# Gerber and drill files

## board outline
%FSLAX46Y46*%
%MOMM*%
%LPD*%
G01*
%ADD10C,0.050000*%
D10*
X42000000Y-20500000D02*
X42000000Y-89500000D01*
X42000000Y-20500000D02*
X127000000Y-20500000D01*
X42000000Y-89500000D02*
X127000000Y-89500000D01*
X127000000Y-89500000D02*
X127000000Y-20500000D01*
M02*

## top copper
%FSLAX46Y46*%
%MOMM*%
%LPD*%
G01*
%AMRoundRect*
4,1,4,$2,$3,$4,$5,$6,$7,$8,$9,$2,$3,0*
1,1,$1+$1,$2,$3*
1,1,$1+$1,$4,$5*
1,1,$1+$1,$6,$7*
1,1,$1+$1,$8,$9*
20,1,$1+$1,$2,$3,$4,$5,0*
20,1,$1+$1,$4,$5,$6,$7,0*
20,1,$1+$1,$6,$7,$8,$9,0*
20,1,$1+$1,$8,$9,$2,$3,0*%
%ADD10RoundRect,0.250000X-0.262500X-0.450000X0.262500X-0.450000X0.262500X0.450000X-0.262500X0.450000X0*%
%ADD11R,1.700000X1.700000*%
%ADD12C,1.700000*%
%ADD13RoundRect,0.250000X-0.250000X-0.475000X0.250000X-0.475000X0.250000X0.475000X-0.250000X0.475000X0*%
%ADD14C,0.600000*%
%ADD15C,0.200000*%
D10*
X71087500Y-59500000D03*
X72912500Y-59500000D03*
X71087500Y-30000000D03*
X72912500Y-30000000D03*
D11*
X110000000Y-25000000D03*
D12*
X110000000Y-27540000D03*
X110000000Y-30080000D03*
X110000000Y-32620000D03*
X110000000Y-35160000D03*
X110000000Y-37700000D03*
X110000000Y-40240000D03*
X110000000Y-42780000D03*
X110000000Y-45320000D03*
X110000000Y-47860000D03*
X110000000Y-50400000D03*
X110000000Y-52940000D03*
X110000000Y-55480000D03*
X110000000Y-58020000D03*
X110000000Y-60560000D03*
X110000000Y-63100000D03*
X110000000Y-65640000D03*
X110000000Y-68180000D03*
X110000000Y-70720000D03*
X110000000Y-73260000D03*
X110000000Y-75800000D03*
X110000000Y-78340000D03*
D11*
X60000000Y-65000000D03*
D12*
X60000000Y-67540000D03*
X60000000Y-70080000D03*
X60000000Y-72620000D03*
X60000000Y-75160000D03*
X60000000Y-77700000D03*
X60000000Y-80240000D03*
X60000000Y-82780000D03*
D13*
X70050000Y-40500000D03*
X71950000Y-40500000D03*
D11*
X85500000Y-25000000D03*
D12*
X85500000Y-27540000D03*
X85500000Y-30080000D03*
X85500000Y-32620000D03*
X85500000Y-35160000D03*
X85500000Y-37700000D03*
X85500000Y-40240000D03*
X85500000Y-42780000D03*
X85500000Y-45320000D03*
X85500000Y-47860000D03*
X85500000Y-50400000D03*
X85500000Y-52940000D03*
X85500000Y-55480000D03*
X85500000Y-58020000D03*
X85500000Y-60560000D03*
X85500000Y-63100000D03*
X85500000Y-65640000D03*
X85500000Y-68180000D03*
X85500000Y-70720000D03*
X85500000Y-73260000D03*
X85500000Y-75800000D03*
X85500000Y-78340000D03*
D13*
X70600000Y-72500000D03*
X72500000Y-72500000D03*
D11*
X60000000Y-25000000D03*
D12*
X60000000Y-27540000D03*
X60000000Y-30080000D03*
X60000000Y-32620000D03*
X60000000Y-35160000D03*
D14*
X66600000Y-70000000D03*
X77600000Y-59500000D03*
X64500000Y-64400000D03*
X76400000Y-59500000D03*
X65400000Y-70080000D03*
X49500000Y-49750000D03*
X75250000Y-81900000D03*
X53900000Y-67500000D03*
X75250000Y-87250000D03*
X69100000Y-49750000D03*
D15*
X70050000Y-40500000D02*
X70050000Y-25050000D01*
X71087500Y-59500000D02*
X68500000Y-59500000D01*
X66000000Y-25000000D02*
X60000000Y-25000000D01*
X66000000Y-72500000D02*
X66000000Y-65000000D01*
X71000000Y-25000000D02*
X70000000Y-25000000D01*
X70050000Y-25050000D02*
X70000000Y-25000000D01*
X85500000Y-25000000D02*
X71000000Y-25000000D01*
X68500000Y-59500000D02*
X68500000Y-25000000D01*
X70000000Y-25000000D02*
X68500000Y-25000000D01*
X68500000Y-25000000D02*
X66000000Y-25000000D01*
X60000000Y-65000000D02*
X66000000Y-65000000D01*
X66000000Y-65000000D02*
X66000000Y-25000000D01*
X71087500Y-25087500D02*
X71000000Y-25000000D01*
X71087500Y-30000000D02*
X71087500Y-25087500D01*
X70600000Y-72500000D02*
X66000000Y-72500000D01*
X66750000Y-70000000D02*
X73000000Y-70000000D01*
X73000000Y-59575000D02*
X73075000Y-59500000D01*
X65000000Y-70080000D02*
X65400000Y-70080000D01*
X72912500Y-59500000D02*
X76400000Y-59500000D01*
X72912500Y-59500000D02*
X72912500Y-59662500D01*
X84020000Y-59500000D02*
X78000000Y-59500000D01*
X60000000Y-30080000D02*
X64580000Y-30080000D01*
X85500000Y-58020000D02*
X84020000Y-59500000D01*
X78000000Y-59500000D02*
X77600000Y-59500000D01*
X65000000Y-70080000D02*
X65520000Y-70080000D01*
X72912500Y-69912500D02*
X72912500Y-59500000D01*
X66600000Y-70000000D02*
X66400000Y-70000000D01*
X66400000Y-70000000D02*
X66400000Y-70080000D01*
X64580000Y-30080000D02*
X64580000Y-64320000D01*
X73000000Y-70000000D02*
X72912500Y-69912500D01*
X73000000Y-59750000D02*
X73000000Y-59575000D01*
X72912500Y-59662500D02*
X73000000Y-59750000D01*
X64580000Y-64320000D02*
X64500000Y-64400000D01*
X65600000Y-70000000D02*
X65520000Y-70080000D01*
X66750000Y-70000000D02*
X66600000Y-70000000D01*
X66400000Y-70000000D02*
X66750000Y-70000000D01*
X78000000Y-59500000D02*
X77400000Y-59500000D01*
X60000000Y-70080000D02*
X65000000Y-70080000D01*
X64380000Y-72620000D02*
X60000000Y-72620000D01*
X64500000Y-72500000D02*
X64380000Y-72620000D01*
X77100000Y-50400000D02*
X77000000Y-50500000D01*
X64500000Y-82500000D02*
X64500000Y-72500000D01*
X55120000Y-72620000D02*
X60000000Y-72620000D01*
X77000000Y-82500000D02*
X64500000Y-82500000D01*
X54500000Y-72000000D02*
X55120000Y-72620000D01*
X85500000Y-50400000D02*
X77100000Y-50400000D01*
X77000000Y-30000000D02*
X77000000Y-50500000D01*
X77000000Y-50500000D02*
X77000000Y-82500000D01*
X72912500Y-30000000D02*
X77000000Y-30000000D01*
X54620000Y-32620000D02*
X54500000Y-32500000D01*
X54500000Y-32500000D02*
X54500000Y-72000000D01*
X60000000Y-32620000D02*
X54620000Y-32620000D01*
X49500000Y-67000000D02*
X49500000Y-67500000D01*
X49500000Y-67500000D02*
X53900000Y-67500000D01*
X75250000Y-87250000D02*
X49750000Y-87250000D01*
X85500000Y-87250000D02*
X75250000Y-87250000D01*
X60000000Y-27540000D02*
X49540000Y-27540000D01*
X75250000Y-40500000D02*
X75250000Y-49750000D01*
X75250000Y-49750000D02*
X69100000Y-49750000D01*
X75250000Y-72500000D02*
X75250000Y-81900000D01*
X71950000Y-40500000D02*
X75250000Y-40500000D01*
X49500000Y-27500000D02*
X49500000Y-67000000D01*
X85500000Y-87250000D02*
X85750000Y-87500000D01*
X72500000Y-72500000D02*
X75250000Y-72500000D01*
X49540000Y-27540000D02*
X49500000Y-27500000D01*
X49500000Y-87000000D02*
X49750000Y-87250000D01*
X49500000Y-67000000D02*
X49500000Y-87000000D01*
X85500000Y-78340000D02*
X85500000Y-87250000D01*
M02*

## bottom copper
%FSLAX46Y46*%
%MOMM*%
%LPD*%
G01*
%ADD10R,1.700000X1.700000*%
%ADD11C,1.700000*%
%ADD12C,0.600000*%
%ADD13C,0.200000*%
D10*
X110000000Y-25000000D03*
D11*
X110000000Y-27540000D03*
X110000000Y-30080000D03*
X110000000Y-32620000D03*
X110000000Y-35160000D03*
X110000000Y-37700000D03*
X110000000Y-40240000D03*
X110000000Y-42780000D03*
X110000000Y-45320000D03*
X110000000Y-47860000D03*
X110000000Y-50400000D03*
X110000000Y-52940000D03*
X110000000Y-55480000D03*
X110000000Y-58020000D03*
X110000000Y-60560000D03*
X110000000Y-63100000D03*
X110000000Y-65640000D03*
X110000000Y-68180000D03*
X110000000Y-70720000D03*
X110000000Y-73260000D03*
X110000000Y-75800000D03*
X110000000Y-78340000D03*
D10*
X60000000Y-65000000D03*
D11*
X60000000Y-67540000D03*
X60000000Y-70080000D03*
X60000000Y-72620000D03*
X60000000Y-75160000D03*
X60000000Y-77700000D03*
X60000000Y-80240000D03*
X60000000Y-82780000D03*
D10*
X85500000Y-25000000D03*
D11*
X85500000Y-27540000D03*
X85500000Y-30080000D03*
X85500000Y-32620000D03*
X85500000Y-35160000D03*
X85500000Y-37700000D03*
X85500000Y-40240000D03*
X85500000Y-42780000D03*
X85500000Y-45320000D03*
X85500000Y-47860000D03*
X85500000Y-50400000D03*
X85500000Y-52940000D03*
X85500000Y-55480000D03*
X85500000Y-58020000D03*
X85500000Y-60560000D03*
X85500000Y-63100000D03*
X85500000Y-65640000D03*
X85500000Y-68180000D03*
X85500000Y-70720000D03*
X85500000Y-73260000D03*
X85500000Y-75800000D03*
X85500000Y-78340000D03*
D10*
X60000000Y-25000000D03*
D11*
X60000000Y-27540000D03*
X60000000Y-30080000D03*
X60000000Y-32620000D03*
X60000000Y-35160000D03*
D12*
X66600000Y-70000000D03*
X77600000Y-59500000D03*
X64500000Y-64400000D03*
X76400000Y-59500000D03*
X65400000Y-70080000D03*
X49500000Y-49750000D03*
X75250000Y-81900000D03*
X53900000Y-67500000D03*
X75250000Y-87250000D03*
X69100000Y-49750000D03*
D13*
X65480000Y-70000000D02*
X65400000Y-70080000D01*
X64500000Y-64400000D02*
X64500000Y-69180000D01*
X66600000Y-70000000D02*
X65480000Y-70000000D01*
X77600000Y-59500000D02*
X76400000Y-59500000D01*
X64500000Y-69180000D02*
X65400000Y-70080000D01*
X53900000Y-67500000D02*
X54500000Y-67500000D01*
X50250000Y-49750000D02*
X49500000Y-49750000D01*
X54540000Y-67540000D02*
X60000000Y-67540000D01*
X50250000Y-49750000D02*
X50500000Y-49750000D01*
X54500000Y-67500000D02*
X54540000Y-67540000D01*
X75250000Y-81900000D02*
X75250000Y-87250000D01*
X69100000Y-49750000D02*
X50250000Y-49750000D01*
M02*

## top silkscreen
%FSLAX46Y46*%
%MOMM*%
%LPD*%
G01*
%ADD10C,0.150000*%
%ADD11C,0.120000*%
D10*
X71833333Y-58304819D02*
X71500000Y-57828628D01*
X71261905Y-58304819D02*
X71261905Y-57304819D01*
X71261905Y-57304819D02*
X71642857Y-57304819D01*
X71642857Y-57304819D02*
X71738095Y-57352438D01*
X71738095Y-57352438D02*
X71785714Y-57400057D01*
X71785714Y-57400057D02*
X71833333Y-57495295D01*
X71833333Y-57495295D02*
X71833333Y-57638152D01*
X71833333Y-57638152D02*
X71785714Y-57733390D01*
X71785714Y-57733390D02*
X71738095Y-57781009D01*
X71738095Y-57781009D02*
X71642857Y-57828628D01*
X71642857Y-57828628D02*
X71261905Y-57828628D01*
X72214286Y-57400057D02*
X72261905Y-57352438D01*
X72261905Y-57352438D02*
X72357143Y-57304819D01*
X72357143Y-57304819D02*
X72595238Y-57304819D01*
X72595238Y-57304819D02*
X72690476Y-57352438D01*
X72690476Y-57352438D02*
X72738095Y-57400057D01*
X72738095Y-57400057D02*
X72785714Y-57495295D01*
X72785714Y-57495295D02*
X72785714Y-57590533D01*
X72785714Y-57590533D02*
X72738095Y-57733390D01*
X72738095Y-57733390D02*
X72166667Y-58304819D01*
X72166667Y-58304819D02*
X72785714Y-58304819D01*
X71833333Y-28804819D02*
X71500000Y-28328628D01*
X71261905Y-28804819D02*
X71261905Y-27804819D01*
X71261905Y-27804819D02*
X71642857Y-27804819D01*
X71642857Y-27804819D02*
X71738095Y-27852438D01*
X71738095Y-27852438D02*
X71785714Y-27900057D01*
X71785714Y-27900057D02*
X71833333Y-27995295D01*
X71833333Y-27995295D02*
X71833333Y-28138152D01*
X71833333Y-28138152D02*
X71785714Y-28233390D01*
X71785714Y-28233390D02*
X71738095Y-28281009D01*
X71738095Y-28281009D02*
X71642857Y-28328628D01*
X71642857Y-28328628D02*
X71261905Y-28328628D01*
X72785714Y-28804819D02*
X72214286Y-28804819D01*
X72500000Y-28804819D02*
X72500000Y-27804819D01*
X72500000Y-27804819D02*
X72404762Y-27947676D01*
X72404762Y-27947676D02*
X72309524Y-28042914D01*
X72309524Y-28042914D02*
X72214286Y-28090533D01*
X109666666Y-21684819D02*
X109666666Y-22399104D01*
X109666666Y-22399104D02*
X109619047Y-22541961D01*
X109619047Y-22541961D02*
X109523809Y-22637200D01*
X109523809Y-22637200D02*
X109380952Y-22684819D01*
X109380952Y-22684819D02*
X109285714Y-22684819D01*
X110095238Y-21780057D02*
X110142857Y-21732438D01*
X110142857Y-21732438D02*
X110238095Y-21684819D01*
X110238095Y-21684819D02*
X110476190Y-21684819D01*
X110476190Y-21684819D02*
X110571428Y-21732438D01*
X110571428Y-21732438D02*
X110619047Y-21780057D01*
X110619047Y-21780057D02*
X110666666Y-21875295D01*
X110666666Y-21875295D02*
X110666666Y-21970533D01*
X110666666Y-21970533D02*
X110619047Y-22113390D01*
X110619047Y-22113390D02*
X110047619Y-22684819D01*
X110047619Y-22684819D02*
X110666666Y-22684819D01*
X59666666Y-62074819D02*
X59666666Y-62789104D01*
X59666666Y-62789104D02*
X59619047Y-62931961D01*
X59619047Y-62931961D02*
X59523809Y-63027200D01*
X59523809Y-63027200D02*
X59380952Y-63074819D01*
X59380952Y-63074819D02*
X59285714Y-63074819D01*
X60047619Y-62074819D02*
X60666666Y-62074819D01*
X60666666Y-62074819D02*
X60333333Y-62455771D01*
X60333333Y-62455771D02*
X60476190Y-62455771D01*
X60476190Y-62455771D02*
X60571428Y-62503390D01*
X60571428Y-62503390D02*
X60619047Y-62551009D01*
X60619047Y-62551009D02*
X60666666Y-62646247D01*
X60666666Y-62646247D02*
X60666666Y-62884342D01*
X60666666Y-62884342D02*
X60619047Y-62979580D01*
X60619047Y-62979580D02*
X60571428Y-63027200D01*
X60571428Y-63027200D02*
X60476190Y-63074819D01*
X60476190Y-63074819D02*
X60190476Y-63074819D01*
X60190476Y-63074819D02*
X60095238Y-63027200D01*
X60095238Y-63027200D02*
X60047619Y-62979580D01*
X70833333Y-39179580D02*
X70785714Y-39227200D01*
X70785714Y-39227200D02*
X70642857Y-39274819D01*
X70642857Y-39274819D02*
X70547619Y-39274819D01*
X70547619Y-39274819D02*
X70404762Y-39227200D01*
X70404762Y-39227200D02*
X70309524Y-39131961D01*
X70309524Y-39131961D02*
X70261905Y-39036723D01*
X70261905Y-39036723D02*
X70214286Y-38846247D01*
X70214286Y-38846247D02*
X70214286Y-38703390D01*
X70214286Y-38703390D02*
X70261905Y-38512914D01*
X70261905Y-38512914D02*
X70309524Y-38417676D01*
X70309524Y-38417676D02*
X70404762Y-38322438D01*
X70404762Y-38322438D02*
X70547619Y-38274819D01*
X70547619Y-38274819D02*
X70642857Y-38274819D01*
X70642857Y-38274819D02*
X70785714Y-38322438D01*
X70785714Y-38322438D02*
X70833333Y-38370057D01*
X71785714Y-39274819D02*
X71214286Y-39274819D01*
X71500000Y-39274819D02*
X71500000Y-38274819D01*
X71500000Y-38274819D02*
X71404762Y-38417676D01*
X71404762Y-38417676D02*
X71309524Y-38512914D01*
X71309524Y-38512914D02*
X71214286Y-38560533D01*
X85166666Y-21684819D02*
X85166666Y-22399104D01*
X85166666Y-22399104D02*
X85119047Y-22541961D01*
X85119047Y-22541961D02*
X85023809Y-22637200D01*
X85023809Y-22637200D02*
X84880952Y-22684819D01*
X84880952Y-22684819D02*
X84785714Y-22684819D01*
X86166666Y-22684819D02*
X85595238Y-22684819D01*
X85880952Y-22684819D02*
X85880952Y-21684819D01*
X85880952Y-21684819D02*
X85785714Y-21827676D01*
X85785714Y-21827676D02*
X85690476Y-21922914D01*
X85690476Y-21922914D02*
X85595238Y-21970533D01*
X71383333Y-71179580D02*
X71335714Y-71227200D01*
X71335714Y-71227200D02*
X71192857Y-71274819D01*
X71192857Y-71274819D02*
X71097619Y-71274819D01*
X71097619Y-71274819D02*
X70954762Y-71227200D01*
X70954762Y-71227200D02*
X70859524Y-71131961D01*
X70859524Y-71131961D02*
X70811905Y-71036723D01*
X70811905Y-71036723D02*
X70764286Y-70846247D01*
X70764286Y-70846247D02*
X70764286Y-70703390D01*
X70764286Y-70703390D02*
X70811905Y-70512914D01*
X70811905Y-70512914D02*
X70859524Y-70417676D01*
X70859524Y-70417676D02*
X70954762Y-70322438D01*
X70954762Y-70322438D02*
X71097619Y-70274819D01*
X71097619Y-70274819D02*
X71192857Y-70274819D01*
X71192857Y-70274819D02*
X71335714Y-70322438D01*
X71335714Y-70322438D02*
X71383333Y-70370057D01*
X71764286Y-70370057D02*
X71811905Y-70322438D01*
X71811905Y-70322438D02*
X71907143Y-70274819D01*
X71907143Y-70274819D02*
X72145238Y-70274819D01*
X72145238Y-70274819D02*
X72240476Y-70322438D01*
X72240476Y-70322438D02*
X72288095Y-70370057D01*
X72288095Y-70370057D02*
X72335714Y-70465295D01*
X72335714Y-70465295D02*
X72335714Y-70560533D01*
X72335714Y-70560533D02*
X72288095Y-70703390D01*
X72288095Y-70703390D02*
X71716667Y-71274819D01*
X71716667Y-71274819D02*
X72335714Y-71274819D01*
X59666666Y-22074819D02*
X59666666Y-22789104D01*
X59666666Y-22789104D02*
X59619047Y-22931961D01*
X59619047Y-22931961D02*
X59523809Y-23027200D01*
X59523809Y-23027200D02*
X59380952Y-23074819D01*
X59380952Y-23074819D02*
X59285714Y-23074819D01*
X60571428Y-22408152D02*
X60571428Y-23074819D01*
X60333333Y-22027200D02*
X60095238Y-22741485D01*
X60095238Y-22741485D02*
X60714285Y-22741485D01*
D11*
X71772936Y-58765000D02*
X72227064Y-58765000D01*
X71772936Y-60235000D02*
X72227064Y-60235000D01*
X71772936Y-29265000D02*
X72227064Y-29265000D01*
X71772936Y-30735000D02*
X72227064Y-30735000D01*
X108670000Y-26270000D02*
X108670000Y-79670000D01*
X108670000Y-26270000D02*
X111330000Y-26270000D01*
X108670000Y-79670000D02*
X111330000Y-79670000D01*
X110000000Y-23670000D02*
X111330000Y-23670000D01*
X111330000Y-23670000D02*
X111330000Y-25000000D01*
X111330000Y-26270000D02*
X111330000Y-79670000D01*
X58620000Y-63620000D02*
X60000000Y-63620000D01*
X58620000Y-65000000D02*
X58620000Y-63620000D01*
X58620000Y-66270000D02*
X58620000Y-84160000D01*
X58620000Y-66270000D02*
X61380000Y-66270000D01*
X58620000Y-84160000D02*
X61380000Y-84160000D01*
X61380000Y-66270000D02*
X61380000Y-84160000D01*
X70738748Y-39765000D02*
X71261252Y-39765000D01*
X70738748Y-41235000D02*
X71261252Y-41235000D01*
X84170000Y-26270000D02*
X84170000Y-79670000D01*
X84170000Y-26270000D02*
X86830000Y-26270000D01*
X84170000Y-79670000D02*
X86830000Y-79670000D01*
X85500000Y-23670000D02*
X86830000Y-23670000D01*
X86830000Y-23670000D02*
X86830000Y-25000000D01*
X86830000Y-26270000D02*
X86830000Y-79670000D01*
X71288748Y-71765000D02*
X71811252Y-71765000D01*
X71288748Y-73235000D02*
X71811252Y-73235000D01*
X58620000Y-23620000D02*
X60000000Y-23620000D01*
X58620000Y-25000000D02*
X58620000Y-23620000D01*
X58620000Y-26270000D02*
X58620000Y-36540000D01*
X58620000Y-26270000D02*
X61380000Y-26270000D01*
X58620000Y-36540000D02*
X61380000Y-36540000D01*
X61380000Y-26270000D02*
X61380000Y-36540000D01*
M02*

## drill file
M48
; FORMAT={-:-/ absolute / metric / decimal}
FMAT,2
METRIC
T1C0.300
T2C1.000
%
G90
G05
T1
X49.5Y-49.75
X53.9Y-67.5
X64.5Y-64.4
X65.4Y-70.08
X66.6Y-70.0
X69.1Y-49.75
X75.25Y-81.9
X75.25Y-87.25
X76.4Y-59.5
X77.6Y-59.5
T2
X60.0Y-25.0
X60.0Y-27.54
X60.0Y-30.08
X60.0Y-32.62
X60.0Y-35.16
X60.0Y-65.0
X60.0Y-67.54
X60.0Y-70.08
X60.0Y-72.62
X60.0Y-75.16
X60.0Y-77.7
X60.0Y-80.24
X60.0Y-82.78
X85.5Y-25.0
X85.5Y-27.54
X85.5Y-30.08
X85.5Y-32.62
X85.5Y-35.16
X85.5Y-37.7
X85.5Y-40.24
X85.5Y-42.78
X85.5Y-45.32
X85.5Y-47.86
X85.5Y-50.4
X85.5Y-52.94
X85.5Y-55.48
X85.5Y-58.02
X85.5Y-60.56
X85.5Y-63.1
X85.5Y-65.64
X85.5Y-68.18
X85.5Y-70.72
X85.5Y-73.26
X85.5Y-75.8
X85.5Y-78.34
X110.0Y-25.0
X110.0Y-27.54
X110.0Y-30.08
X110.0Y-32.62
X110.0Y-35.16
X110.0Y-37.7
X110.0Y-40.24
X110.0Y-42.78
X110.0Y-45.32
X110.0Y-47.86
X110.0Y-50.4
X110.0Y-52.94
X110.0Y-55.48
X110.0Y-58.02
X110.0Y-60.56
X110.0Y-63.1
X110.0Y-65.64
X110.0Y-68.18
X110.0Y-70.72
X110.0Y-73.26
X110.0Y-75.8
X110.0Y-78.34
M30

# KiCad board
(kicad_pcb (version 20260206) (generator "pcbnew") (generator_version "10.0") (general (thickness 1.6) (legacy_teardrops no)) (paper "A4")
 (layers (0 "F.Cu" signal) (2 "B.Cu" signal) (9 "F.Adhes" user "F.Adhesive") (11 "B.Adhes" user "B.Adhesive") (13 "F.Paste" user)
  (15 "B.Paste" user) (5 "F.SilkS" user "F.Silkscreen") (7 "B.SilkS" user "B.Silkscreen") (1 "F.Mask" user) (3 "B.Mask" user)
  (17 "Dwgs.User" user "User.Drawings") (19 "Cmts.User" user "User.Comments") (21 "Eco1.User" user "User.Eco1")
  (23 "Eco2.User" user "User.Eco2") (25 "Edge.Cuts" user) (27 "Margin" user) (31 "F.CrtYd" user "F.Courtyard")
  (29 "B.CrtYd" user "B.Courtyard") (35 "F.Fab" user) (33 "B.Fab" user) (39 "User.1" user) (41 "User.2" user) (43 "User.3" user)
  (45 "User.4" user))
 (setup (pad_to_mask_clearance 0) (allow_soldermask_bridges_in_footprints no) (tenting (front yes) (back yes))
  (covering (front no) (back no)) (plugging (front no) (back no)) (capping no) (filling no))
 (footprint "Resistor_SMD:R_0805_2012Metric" (layer "F.Cu") (at 72 59.5)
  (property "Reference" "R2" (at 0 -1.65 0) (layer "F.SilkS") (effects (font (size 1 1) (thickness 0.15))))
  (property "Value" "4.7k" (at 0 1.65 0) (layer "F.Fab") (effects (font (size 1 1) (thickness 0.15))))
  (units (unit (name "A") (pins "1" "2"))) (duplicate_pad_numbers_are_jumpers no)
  (fp_line (start -0.227064 -0.735) (end 0.227064 -0.735) (stroke (width 0.12) (type solid)) (layer "F.SilkS"))
  (fp_line (start -0.227064 0.735) (end 0.227064 0.735) (stroke (width 0.12) (type solid)) (layer "F.SilkS"))
  (pad "1" smd roundrect (at -0.9125 0) (size 1.025 1.4) (layers "F.Cu" "F.Mask" "F.Paste") (roundrect_rratio 0.243902) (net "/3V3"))
  (pad "2" smd roundrect (at 0.9125 0) (size 1.025 1.4) (layers "F.Cu" "F.Mask" "F.Paste") (roundrect_rratio 0.243902) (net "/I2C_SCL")))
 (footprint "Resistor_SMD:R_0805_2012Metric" (layer "F.Cu") (at 72 30)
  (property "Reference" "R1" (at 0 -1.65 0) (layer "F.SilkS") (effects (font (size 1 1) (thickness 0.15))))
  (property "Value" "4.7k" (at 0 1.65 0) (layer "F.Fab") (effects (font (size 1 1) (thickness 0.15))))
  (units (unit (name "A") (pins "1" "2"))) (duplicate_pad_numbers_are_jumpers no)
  (fp_line (start -0.227064 -0.735) (end 0.227064 -0.735) (stroke (width 0.12) (type solid)) (layer "F.SilkS"))
  (fp_line (start -0.227064 0.735) (end 0.227064 0.735) (stroke (width 0.12) (type solid)) (layer "F.SilkS"))
  (pad "1" smd roundrect (at -0.9125 0) (size 1.025 1.4) (layers "F.Cu" "F.Mask" "F.Paste") (roundrect_rratio 0.243902) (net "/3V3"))
  (pad "2" smd roundrect (at 0.9125 0) (size 1.025 1.4) (layers "F.Cu" "F.Mask" "F.Paste") (roundrect_rratio 0.243902) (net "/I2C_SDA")))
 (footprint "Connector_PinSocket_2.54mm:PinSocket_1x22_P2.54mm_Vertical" (layer "F.Cu") (at 110 25)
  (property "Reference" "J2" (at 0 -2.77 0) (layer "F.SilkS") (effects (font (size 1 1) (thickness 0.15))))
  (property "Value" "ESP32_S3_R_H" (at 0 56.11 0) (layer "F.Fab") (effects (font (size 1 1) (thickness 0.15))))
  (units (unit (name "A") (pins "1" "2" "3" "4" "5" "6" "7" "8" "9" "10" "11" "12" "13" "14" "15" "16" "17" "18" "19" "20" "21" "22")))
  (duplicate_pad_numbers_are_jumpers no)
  (fp_line (start -1.33 1.27) (end -1.33 54.67) (stroke (width 0.12) (type solid)) (layer "F.SilkS"))
  (fp_line (start -1.33 1.27) (end 1.33 1.27) (stroke (width 0.12) (type solid)) (layer "F.SilkS"))
  (fp_line (start -1.33 54.67) (end 1.33 54.67) (stroke (width 0.12) (type solid)) (layer "F.SilkS"))
  (fp_line (start 0 -1.33) (end 1.33 -1.33) (stroke (width 0.12) (type solid)) (layer "F.SilkS"))
  (fp_line (start 1.33 -1.33) (end 1.33 0) (stroke (width 0.12) (type solid)) (layer "F.SilkS"))
  (fp_line (start 1.33 1.27) (end 1.33 54.67) (stroke (width 0.12) (type solid)) (layer "F.SilkS"))
  (pad "1" thru_hole rect (at 0 0) (size 1.7 1.7) (drill 1) (layers "*.Cu" "*.Mask") (remove_unused_layers no) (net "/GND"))
  (pad "2" thru_hole circle (at 0 2.54) (size 1.7 1.7) (drill 1) (layers "*.Cu" "*.Mask") (remove_unused_layers no)
   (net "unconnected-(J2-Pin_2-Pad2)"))
  (pad "3" thru_hole circle (at 0 5.08) (size 1.7 1.7) (drill 1) (layers "*.Cu" "*.Mask") (remove_unused_layers no)
   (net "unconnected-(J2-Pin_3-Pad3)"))
  (pad "4" thru_hole circle (at 0 7.62) (size 1.7 1.7) (drill 1) (layers "*.Cu" "*.Mask") (remove_unused_layers no)
   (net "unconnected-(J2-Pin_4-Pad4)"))
  (pad "5" thru_hole circle (at 0 10.16) (size 1.7 1.7) (drill 1) (layers "*.Cu" "*.Mask") (remove_unused_layers no)
   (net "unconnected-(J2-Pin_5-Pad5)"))
  (pad "6" thru_hole circle (at 0 12.7) (size 1.7 1.7) (drill 1) (layers "*.Cu" "*.Mask") (remove_unused_layers no)
   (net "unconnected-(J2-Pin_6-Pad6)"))
  (pad "7" thru_hole circle (at 0 15.24) (size 1.7 1.7) (drill 1) (layers "*.Cu" "*.Mask") (remove_unused_layers no)
   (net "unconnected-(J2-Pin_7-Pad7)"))
  (pad "8" thru_hole circle (at 0 17.78) (size 1.7 1.7) (drill 1) (layers "*.Cu" "*.Mask") (remove_unused_layers no)
   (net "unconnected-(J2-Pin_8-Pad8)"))
  (pad "9" thru_hole circle (at 0 20.32) (size 1.7 1.7) (drill 1) (layers "*.Cu" "*.Mask") (remove_unused_layers no)
   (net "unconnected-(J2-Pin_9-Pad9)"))
  (pad "10" thru_hole circle (at 0 22.86) (size 1.7 1.7) (drill 1) (layers "*.Cu" "*.Mask") (remove_unused_layers no)
   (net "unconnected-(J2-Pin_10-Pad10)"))
  (pad "11" thru_hole circle (at 0 25.4) (size 1.7 1.7) (drill 1) (layers "*.Cu" "*.Mask") (remove_unused_layers no)
   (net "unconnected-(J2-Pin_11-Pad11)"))
  (pad "12" thru_hole circle (at 0 27.94) (size 1.7 1.7) (drill 1) (layers "*.Cu" "*.Mask") (remove_unused_layers no)
   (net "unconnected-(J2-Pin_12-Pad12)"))
  (pad "13" thru_hole circle (at 0 30.48) (size 1.7 1.7) (drill 1) (layers "*.Cu" "*.Mask") (remove_unused_layers no)
   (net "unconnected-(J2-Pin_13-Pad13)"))
  (pad "14" thru_hole circle (at 0 33.02) (size 1.7 1.7) (drill 1) (layers "*.Cu" "*.Mask") (remove_unused_layers no)
   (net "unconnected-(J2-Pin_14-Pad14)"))
  (pad "15" thru_hole circle (at 0 35.56) (size 1.7 1.7) (drill 1) (layers "*.Cu" "*.Mask") (remove_unused_layers no)
   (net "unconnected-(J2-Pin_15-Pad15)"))
  (pad "16" thru_hole circle (at 0 38.1) (size 1.7 1.7) (drill 1) (layers "*.Cu" "*.Mask") (remove_unused_layers no)
   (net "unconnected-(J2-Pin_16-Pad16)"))
  (pad "17" thru_hole circle (at 0 40.64) (size 1.7 1.7) (drill 1) (layers "*.Cu" "*.Mask") (remove_unused_layers no)
   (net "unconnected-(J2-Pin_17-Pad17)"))
  (pad "18" thru_hole circle (at 0 43.18) (size 1.7 1.7) (drill 1) (layers "*.Cu" "*.Mask") (remove_unused_layers no)
   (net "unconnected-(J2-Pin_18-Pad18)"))
  (pad "19" thru_hole circle (at 0 45.72) (size 1.7 1.7) (drill 1) (layers "*.Cu" "*.Mask") (remove_unused_layers no)
   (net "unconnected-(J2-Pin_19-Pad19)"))
  (pad "20" thru_hole circle (at 0 48.26) (size 1.7 1.7) (drill 1) (layers "*.Cu" "*.Mask") (remove_unused_layers no)
   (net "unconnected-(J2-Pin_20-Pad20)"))
  (pad "21" thru_hole circle (at 0 50.8) (size 1.7 1.7) (drill 1) (layers "*.Cu" "*.Mask") (remove_unused_layers no) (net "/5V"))
  (pad "22" thru_hole circle (at 0 53.34) (size 1.7 1.7) (drill 1) (layers "*.Cu" "*.Mask") (remove_unused_layers no) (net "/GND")))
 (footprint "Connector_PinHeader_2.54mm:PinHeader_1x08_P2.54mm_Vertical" (layer "F.Cu") (at 60 65)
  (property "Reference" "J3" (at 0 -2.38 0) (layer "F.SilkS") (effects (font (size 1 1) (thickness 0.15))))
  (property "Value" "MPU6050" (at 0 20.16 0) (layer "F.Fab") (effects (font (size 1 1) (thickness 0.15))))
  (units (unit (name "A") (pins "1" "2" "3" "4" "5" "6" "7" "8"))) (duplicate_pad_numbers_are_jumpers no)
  (fp_line (start -1.38 -1.38) (end 0 -1.38) (stroke (width 0.12) (type solid)) (layer "F.SilkS"))
  (fp_line (start -1.38 0) (end -1.38 -1.38) (stroke (width 0.12) (type solid)) (layer "F.SilkS"))
  (fp_line (start -1.38 1.27) (end -1.38 19.16) (stroke (width 0.12) (type solid)) (layer "F.SilkS"))
  (fp_line (start -1.38 1.27) (end 1.38 1.27) (stroke (width 0.12) (type solid)) (layer "F.SilkS"))
  (fp_line (start -1.38 19.16) (end 1.38 19.16) (stroke (width 0.12) (type solid)) (layer "F.SilkS"))
  (fp_line (start 1.38 1.27) (end 1.38 19.16) (stroke (width 0.12) (type solid)) (layer "F.SilkS"))
  (pad "1" thru_hole rect (at 0 0) (size 1.7 1.7) (drill 1) (layers "*.Cu" "*.Mask") (remove_unused_layers no) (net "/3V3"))
  (pad "2" thru_hole circle (at 0 2.54) (size 1.7 1.7) (drill 1) (layers "*.Cu" "*.Mask") (remove_unused_layers no) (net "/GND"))
  (pad "3" thru_hole circle (at 0 5.08) (size 1.7 1.7) (drill 1) (layers "*.Cu" "*.Mask") (remove_unused_layers no) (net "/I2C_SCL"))
  (pad "4" thru_hole circle (at 0 7.62) (size 1.7 1.7) (drill 1) (layers "*.Cu" "*.Mask") (remove_unused_layers no) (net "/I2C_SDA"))
  (pad "5" thru_hole circle (at 0 10.16) (size 1.7 1.7) (drill 1) (layers "*.Cu" "*.Mask") (remove_unused_layers no)
   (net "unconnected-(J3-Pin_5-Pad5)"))
  (pad "6" thru_hole circle (at 0 12.7) (size 1.7 1.7) (drill 1) (layers "*.Cu" "*.Mask") (remove_unused_layers no)
   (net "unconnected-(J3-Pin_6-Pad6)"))
  (pad "7" thru_hole circle (at 0 15.24) (size 1.7 1.7) (drill 1) (layers "*.Cu" "*.Mask") (remove_unused_layers no) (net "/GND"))
  (pad "8" thru_hole circle (at 0 17.78) (size 1.7 1.7) (drill 1) (layers "*.Cu" "*.Mask") (remove_unused_layers no) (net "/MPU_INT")))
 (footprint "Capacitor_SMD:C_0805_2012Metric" (layer "F.Cu") (at 71 40.5)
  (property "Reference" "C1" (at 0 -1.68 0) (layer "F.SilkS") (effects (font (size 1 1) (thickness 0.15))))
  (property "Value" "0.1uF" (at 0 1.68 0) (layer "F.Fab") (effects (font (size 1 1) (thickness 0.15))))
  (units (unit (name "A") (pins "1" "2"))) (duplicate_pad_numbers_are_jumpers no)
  (fp_line (start -0.261252 -0.735) (end 0.261252 -0.735) (stroke (width 0.12) (type solid)) (layer "F.SilkS"))
  (fp_line (start -0.261252 0.735) (end 0.261252 0.735) (stroke (width 0.12) (type solid)) (layer "F.SilkS"))
  (pad "1" smd roundrect (at -0.95 0) (size 1 1.45) (layers "F.Cu" "F.Mask" "F.Paste") (roundrect_rratio 0.25) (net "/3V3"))
  (pad "2" smd roundrect (at 0.95 0) (size 1 1.45) (layers "F.Cu" "F.Mask" "F.Paste") (roundrect_rratio 0.25) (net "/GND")))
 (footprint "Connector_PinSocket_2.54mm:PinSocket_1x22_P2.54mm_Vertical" (layer "F.Cu") (at 85.5 25)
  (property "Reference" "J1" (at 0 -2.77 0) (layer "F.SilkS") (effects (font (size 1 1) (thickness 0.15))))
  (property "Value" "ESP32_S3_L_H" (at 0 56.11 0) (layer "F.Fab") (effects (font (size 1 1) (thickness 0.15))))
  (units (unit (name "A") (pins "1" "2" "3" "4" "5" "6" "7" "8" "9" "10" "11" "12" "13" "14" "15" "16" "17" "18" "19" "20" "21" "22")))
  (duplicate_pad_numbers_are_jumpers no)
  (fp_line (start -1.33 1.27) (end -1.33 54.67) (stroke (width 0.12) (type solid)) (layer "F.SilkS"))
  (fp_line (start -1.33 1.27) (end 1.33 1.27) (stroke (width 0.12) (type solid)) (layer "F.SilkS"))
  (fp_line (start -1.33 54.67) (end 1.33 54.67) (stroke (width 0.12) (type solid)) (layer "F.SilkS"))
  (fp_line (start 0 -1.33) (end 1.33 -1.33) (stroke (width 0.12) (type solid)) (layer "F.SilkS"))
  (fp_line (start 1.33 -1.33) (end 1.33 0) (stroke (width 0.12) (type solid)) (layer "F.SilkS"))
  (fp_line (start 1.33 1.27) (end 1.33 54.67) (stroke (width 0.12) (type solid)) (layer "F.SilkS"))
  (pad "1" thru_hole rect (at 0 0) (size 1.7 1.7) (drill 1) (layers "*.Cu" "*.Mask") (remove_unused_layers no) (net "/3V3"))
  (pad "2" thru_hole circle (at 0 2.54) (size 1.7 1.7) (drill 1) (layers "*.Cu" "*.Mask") (remove_unused_layers no)
   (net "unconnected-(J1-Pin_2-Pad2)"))
  (pad "3" thru_hole circle (at 0 5.08) (size 1.7 1.7) (drill 1) (layers "*.Cu" "*.Mask") (remove_unused_layers no)
   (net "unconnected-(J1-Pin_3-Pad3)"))
  (pad "4" thru_hole circle (at 0 7.62) (size 1.7 1.7) (drill 1) (layers "*.Cu" "*.Mask") (remove_unused_layers no)
   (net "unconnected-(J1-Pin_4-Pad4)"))
  (pad "5" thru_hole circle (at 0 10.16) (size 1.7 1.7) (drill 1) (layers "*.Cu" "*.Mask") (remove_unused_layers no)
   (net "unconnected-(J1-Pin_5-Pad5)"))
  (pad "6" thru_hole circle (at 0 12.7) (size 1.7 1.7) (drill 1) (layers "*.Cu" "*.Mask") (remove_unused_layers no)
   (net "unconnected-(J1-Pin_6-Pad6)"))
  (pad "7" thru_hole circle (at 0 15.24) (size 1.7 1.7) (drill 1) (layers "*.Cu" "*.Mask") (remove_unused_layers no)
   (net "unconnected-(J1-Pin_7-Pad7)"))
  (pad "8" thru_hole circle (at 0 17.78) (size 1.7 1.7) (drill 1) (layers "*.Cu" "*.Mask") (remove_unused_layers no)
   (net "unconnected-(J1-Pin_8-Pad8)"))
  (pad "9" thru_hole circle (at 0 20.32) (size 1.7 1.7) (drill 1) (layers "*.Cu" "*.Mask") (remove_unused_layers no)
   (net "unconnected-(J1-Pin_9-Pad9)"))
  (pad "10" thru_hole circle (at 0 22.86) (size 1.7 1.7) (drill 1) (layers "*.Cu" "*.Mask") (remove_unused_layers no)
   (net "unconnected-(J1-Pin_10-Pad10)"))
  (pad "11" thru_hole circle (at 0 25.4) (size 1.7 1.7) (drill 1) (layers "*.Cu" "*.Mask") (remove_unused_layers no) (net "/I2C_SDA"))
  (pad "12" thru_hole circle (at 0 27.94) (size 1.7 1.7) (drill 1) (layers "*.Cu" "*.Mask") (remove_unused_layers no)
   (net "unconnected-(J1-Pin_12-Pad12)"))
  (pad "13" thru_hole circle (at 0 30.48) (size 1.7 1.7) (drill 1) (layers "*.Cu" "*.Mask") (remove_unused_layers no)
   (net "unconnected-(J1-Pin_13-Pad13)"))
  (pad "14" thru_hole circle (at 0 33.02) (size 1.7 1.7) (drill 1) (layers "*.Cu" "*.Mask") (remove_unused_layers no) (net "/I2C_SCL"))
  (pad "15" thru_hole circle (at 0 35.56) (size 1.7 1.7) (drill 1) (layers "*.Cu" "*.Mask") (remove_unused_layers no) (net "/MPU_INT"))
  (pad "16" thru_hole circle (at 0 38.1) (size 1.7 1.7) (drill 1) (layers "*.Cu" "*.Mask") (remove_unused_layers no) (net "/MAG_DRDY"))
  (pad "17" thru_hole circle (at 0 40.64) (size 1.7 1.7) (drill 1) (layers "*.Cu" "*.Mask") (remove_unused_layers no)
   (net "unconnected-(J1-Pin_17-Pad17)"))
  (pad "18" thru_hole circle (at 0 43.18) (size 1.7 1.7) (drill 1) (layers "*.Cu" "*.Mask") (remove_unused_layers no)
   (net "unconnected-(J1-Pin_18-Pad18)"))
  (pad "19" thru_hole circle (at 0 45.72) (size 1.7 1.7) (drill 1) (layers "*.Cu" "*.Mask") (remove_unused_layers no)
   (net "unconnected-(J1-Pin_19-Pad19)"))
  (pad "20" thru_hole circle (at 0 48.26) (size 1.7 1.7) (drill 1) (layers "*.Cu" "*.Mask") (remove_unused_layers no)
   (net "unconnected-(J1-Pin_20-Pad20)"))
  (pad "21" thru_hole circle (at 0 50.8) (size 1.7 1.7) (drill 1) (layers "*.Cu" "*.Mask") (remove_unused_layers no) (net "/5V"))
  (pad "22" thru_hole circle (at 0 53.34) (size 1.7 1.7) (drill 1) (layers "*.Cu" "*.Mask") (remove_unused_layers no) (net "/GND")))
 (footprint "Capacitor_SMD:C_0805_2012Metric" (layer "F.Cu") (at 71.55 72.5)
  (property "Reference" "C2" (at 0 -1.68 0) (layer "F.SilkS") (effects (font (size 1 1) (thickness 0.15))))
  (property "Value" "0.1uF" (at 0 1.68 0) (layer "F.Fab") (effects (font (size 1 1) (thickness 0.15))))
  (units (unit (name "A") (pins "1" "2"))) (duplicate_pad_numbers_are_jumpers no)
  (fp_line (start -0.261252 -0.735) (end 0.261252 -0.735) (stroke (width 0.12) (type solid)) (layer "F.SilkS"))
  (fp_line (start -0.261252 0.735) (end 0.261252 0.735) (stroke (width 0.12) (type solid)) (layer "F.SilkS"))
  (pad "1" smd roundrect (at -0.95 0) (size 1 1.45) (layers "F.Cu" "F.Mask" "F.Paste") (roundrect_rratio 0.25) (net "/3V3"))
  (pad "2" smd roundrect (at 0.95 0) (size 1 1.45) (layers "F.Cu" "F.Mask" "F.Paste") (roundrect_rratio 0.25) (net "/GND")))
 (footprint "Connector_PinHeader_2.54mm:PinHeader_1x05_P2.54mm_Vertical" (layer "F.Cu") (at 60 25)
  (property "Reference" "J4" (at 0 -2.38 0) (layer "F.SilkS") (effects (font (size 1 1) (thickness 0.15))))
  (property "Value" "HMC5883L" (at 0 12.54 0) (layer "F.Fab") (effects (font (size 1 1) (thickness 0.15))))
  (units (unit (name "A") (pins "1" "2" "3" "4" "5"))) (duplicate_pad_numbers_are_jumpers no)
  (fp_line (start -1.38 -1.38) (end 0 -1.38) (stroke (width 0.12) (type solid)) (layer "F.SilkS"))
  (fp_line (start -1.38 0) (end -1.38 -1.38) (stroke (width 0.12) (type solid)) (layer "F.SilkS"))
  (fp_line (start -1.38 1.27) (end -1.38 11.54) (stroke (width 0.12) (type solid)) (layer "F.SilkS"))
  (fp_line (start -1.38 1.27) (end 1.38 1.27) (stroke (width 0.12) (type solid)) (layer "F.SilkS"))
  (fp_line (start -1.38 11.54) (end 1.38 11.54) (stroke (width 0.12) (type solid)) (layer "F.SilkS"))
  (fp_line (start 1.38 1.27) (end 1.38 11.54) (stroke (width 0.12) (type solid)) (layer "F.SilkS"))
  (pad "1" thru_hole rect (at 0 0) (size 1.7 1.7) (drill 1) (layers "*.Cu" "*.Mask") (remove_unused_layers no) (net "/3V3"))
  (pad "2" thru_hole circle (at 0 2.54) (size 1.7 1.7) (drill 1) (layers "*.Cu" "*.Mask") (remove_unused_layers no) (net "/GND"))
  (pad "3" thru_hole circle (at 0 5.08) (size 1.7 1.7) (drill 1) (layers "*.Cu" "*.Mask") (remove_unused_layers no) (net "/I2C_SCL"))
  (pad "4" thru_hole circle (at 0 7.62) (size 1.7 1.7) (drill 1) (layers "*.Cu" "*.Mask") (remove_unused_layers no) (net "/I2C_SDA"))
  (pad "5" thru_hole circle (at 0 10.16) (size 1.7 1.7) (drill 1) (layers "*.Cu" "*.Mask") (remove_unused_layers no) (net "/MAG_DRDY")))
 (gr_line (start 42 20.5) (end 42 89.5) (stroke (width 0.05) (type default)) (layer "Edge.Cuts"))
 (gr_line (start 42 20.5) (end 127 20.5) (stroke (width 0.05) (type default)) (layer "Edge.Cuts"))
 (gr_line (start 42 89.5) (end 127 89.5) (stroke (width 0.05) (type default)) (layer "Edge.Cuts"))
 (gr_line (start 127 89.5) (end 127 20.5) (stroke (width 0.05) (type default)) (layer "Edge.Cuts"))
 (segment (start 70.05 40.5) (end 70.05 25.05) (width 0.2) (layer "F.Cu") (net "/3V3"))
 (segment (start 71.0875 59.5) (end 68.5 59.5) (width 0.2) (layer "F.Cu") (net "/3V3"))
 (segment (start 66 25) (end 60 25) (width 0.2) (layer "F.Cu") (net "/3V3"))
 (segment (start 66 72.5) (end 66 65) (width 0.2) (layer "F.Cu") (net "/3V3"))
 (segment (start 71 25) (end 70 25) (width 0.2) (layer "F.Cu") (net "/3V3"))
 (segment (start 70.05 25.05) (end 70 25) (width 0.2) (layer "F.Cu") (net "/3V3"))
 (segment (start 85.5 25) (end 71 25) (width 0.2) (layer "F.Cu") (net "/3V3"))
 (segment (start 68.5 59.5) (end 68.5 25) (width 0.2) (layer "F.Cu") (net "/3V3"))
 (segment (start 70 25) (end 68.5 25) (width 0.2) (layer "F.Cu") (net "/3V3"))
 (segment (start 68.5 25) (end 66 25) (width 0.2) (layer "F.Cu") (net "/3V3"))
 (segment (start 60 65) (end 66 65) (width 0.2) (layer "F.Cu") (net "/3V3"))
 (segment (start 66 65) (end 66 25) (width 0.2) (layer "F.Cu") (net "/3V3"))
 (segment (start 71.0875 25.0875) (end 71 25) (width 0.2) (layer "F.Cu") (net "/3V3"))
 (segment (start 71.0875 30) (end 71.0875 25.0875) (width 0.2) (layer "F.Cu") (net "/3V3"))
 (segment (start 70.6 72.5) (end 66 72.5) (width 0.2) (layer "F.Cu") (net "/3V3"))
 (segment (start 66.75 70) (end 73 70) (width 0.2) (layer "F.Cu") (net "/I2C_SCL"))
 (segment (start 73 59.575) (end 73.075 59.5) (width 0.2) (layer "F.Cu") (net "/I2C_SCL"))
 (segment (start 65 70.08) (end 65.4 70.08) (width 0.2) (layer "F.Cu") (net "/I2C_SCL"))
 (segment (start 72.9125 59.5) (end 76.4 59.5) (width 0.2) (layer "F.Cu") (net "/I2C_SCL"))
 (segment (start 72.9125 59.5) (end 72.9125 59.6625) (width 0.2) (layer "F.Cu") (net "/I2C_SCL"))
 (segment (start 84.02 59.5) (end 78 59.5) (width 0.2) (layer "F.Cu") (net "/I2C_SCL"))
 (segment (start 60 30.08) (end 64.58 30.08) (width 0.2) (layer "F.Cu") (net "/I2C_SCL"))
 (segment (start 85.5 58.02) (end 84.02 59.5) (width 0.2) (layer "F.Cu") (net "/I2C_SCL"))
 (segment (start 78 59.5) (end 77.6 59.5) (width 0.2) (layer "F.Cu") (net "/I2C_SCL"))
 (segment (start 65 70.08) (end 65.52 70.08) (width 0.2) (layer "F.Cu") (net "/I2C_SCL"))
 (segment (start 72.9125 69.9125) (end 72.9125 59.5) (width 0.2) (layer "F.Cu") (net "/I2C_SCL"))
 (segment (start 66.6 70) (end 66.4 70) (width 0.2) (layer "F.Cu") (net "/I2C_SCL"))
 (segment (start 66.4 70) (end 66.4 70.08) (width 0.2) (layer "F.Cu") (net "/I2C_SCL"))
 (segment (start 64.58 30.08) (end 64.58 64.32) (width 0.2) (layer "F.Cu") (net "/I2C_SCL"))
 (segment (start 73 70) (end 72.9125 69.9125) (width 0.2) (layer "F.Cu") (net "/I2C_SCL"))
 (segment (start 73 59.75) (end 73 59.575) (width 0.2) (layer "F.Cu") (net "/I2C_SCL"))
 (segment (start 72.9125 59.6625) (end 73 59.75) (width 0.2) (layer "F.Cu") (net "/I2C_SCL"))
 (segment (start 64.58 64.32) (end 64.5 64.4) (width 0.2) (layer "F.Cu") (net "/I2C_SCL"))
 (segment (start 65.6 70) (end 65.52 70.08) (width 0.2) (layer "F.Cu") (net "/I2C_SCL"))
 (segment (start 66.75 70) (end 66.6 70) (width 0.2) (layer "F.Cu") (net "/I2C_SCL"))
 (segment (start 66.4 70) (end 66.75 70) (width 0.2) (layer "F.Cu") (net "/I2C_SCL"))
 (segment (start 78 59.5) (end 77.4 59.5) (width 0.2) (layer "F.Cu") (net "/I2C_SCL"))
 (segment (start 60 70.08) (end 65 70.08) (width 0.2) (layer "F.Cu") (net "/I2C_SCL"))
 (via (at 66.6 70) (size 0.6) (drill 0.3) (layers "F.Cu" "B.Cu") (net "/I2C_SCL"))
 (via (at 77.6 59.5) (size 0.6) (drill 0.3) (layers "F.Cu" "B.Cu") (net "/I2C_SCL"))
 (via (at 64.5 64.4) (size 0.6) (drill 0.3) (layers "F.Cu" "B.Cu") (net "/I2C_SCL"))
 (via (at 76.4 59.5) (size 0.6) (drill 0.3) (layers "F.Cu" "B.Cu") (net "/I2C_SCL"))
 (via (at 65.4 70.08) (size 0.6) (drill 0.3) (layers "F.Cu" "B.Cu") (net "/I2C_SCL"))
 (segment (start 65.48 70) (end 65.4 70.08) (width 0.2) (layer "B.Cu") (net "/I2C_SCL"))
 (segment (start 64.5 64.4) (end 64.5 69.18) (width 0.2) (layer "B.Cu") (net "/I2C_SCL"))
 (segment (start 66.6 70) (end 65.48 70) (width 0.2) (layer "B.Cu") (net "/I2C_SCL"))
 (segment (start 77.6 59.5) (end 76.4 59.5) (width 0.2) (layer "B.Cu") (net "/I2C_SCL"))
 (segment (start 64.5 69.18) (end 65.4 70.08) (width 0.2) (layer "B.Cu") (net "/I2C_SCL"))
 (segment (start 64.38 72.62) (end 60 72.62) (width 0.2) (layer "F.Cu") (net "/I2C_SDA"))
 (segment (start 64.5 72.5) (end 64.38 72.62) (width 0.2) (layer "F.Cu") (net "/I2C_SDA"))
 (segment (start 77.1 50.4) (end 77 50.5) (width 0.2) (layer "F.Cu") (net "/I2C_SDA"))
 (segment (start 64.5 82.5) (end 64.5 72.5) (width 0.2) (layer "F.Cu") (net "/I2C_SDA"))
 (segment (start 55.12 72.62) (end 60 72.62) (width 0.2) (layer "F.Cu") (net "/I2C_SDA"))
 (segment (start 77 82.5) (end 64.5 82.5) (width 0.2) (layer "F.Cu") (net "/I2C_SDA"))
 (segment (start 54.5 72) (end 55.12 72.62) (width 0.2) (layer "F.Cu") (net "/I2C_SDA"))
 (segment (start 85.5 50.4) (end 77.1 50.4) (width 0.2) (layer "F.Cu") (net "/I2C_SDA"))
 (segment (start 77 30) (end 77 50.5) (width 0.2) (layer "F.Cu") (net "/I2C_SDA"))
 (segment (start 77 50.5) (end 77 82.5) (width 0.2) (layer "F.Cu") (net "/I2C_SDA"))
 (segment (start 72.9125 30) (end 77 30) (width 0.2) (layer "F.Cu") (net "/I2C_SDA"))
 (segment (start 54.62 32.62) (end 54.5 32.5) (width 0.2) (layer "F.Cu") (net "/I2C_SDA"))
 (segment (start 54.5 32.5) (end 54.5 72) (width 0.2) (layer "F.Cu") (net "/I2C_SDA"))
 (segment (start 60 32.62) (end 54.62 32.62) (width 0.2) (layer "F.Cu") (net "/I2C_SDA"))
 (segment (start 49.5 67) (end 49.5 67.5) (width 0.2) (layer "F.Cu") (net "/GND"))
 (segment (start 49.5 67.5) (end 53.9 67.5) (width 0.2) (layer "F.Cu") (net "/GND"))
 (segment (start 75.25 87.25) (end 49.75 87.25) (width 0.2) (layer "F.Cu") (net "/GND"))
 (segment (start 85.5 87.25) (end 75.25 87.25) (width 0.2) (layer "F.Cu") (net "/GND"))
 (segment (start 60 27.54) (end 49.54 27.54) (width 0.2) (layer "F.Cu") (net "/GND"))
 (segment (start 75.25 40.5) (end 75.25 49.75) (width 0.2) (layer "F.Cu") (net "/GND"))
 (segment (start 75.25 49.75) (end 69.1 49.75) (width 0.2) (layer "F.Cu") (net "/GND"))
 (segment (start 75.25 72.5) (end 75.25 81.9) (width 0.2) (layer "F.Cu") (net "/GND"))
 (segment (start 71.95 40.5) (end 75.25 40.5) (width 0.2) (layer "F.Cu") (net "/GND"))
 (segment (start 49.5 27.5) (end 49.5 67) (width 0.2) (layer "F.Cu") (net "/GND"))
 (segment (start 85.5 87.25) (end 85.75 87.5) (width 0.2) (layer "F.Cu") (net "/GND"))
 (segment (start 72.5 72.5) (end 75.25 72.5) (width 0.2) (layer "F.Cu") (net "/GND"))
 (segment (start 49.54 27.54) (end 49.5 27.5) (width 0.2) (layer "F.Cu") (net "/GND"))
 (segment (start 49.5 87) (end 49.75 87.25) (width 0.2) (layer "F.Cu") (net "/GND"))
 (segment (start 49.5 67) (end 49.5 87) (width 0.2) (layer "F.Cu") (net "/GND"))
 (segment (start 85.5 78.34) (end 85.5 87.25) (width 0.2) (layer "F.Cu") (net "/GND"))
 (via (at 49.5 49.75) (size 0.6) (drill 0.3) (layers "F.Cu" "B.Cu") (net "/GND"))
 (via (at 75.25 81.9) (size 0.6) (drill 0.3) (layers "F.Cu" "B.Cu") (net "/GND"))
 (via (at 53.9 67.5) (size 0.6) (drill 0.3) (layers "F.Cu" "B.Cu") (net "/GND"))
 (via (at 75.25 87.25) (size 0.6) (drill 0.3) (layers "F.Cu" "B.Cu") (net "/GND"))
 (via (at 69.1 49.75) (size 0.6) (drill 0.3) (layers "F.Cu" "B.Cu") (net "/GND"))
 (segment (start 53.9 67.5) (end 54.5 67.5) (width 0.2) (layer "B.Cu") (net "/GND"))
 (segment (start 50.25 49.75) (end 49.5 49.75) (width 0.2) (layer "B.Cu") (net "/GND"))
 (segment (start 54.54 67.54) (end 60 67.54) (width 0.2) (layer "B.Cu") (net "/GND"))
 (segment (start 50.25 49.75) (end 50.5 49.75) (width 0.2) (layer "B.Cu") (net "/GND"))
 (segment (start 54.5 67.5) (end 54.54 67.54) (width 0.2) (layer "B.Cu") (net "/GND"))
 (segment (start 75.25 81.9) (end 75.25 87.25) (width 0.2) (layer "B.Cu") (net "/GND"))
 (segment (start 69.1 49.75) (end 50.25 49.75) (width 0.2) (layer "B.Cu") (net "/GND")))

